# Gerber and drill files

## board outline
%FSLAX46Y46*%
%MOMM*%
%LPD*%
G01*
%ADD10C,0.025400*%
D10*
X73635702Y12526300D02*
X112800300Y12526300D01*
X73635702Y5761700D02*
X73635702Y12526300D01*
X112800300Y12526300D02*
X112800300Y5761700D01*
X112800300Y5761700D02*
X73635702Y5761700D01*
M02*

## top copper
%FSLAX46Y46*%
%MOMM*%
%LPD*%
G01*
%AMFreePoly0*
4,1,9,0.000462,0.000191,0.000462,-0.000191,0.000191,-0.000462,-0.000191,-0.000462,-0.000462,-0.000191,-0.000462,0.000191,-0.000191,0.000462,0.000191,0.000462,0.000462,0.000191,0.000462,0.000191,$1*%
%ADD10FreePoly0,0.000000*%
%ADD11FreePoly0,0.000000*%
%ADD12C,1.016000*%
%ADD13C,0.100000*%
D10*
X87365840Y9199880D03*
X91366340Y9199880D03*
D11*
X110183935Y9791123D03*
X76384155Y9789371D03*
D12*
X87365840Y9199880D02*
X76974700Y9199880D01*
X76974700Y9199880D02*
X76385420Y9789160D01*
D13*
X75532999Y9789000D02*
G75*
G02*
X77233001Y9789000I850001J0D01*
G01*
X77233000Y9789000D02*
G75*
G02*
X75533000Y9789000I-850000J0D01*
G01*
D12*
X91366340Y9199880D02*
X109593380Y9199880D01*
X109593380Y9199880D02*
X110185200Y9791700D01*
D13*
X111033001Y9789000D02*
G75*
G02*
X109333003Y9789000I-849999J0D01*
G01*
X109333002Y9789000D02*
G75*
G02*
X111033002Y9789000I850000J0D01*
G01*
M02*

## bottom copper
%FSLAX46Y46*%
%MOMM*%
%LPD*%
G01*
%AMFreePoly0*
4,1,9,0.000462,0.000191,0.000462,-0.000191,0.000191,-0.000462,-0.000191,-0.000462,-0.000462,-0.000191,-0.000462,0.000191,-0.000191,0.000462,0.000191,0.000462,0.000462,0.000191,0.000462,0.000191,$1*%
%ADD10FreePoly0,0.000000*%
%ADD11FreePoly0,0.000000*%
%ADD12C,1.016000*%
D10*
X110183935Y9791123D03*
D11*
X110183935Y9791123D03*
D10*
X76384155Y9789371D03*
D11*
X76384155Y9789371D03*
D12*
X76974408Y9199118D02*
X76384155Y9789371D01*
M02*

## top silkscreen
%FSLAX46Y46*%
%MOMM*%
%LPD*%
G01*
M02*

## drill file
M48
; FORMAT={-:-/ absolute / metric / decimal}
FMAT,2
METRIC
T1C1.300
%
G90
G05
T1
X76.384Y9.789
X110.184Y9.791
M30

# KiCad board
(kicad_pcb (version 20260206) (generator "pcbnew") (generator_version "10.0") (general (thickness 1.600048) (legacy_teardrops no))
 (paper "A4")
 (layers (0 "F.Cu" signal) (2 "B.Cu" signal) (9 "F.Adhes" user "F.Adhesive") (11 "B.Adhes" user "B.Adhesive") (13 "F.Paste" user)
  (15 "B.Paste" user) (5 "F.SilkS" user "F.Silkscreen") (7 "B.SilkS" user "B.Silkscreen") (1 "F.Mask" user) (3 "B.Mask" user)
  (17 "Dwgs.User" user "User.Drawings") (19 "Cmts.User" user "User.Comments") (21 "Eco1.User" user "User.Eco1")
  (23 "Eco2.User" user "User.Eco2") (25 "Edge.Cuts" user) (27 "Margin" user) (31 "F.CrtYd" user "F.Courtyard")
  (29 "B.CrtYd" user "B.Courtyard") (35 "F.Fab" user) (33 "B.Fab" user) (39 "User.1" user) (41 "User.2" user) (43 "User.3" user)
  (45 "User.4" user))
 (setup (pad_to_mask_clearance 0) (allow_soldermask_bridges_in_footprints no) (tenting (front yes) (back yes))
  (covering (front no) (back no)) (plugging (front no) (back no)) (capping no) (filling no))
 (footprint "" (layer "F.Cu") (at 0 0)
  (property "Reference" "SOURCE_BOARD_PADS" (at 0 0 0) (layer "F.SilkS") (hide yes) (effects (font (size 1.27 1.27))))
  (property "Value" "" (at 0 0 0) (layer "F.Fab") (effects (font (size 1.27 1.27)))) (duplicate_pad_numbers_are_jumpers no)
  (pad "1" smd custom (at 87.36584 -9.19988) (size 0.001 0.001) (layers "F.Cu" "F.Mask" "F.Paste") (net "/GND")
   (options (clearance outline) (anchor circle)) (primitives))
  (pad "2" smd custom (at 91.36634 -9.19988) (size 0.001 0.001) (layers "F.Cu" "F.Mask" "F.Paste") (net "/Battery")
   (options (clearance outline) (anchor circle)) (primitives)))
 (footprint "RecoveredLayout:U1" (layer "B.Cu") (at 110.183935 -9.791123)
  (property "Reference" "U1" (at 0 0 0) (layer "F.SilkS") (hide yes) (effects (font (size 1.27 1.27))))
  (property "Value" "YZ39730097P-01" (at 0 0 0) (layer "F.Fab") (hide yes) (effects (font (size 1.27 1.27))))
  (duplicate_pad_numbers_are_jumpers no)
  (pad "1" thru_hole custom (at 0 0) (size 0.001 0.001) (drill 1.300023) (layers "*.Cu") (remove_unused_layers no) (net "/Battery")
   (options (clearance outline) (anchor circle)) (primitives))
  (pad "1" smd custom (at 0 0) (size 0.001 0.001) (layers "B.Cu" "B.Mask" "B.Paste") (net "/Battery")
   (options (clearance outline) (anchor circle)) (primitives)))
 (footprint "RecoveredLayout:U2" (layer "B.Cu") (at 76.384155 -9.789371)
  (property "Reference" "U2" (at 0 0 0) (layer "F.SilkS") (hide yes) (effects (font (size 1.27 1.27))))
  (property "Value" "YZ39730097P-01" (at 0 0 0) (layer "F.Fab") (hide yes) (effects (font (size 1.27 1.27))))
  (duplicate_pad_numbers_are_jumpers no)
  (pad "1" thru_hole custom (at 0 0) (size 0.001 0.001) (drill 1.300023) (layers "*.Cu") (remove_unused_layers no) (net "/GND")
   (options (clearance outline) (anchor circle)) (primitives))
  (pad "1" smd custom (at 0 0) (size 0.001 0.001) (layers "B.Cu" "B.Mask" "B.Paste") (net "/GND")
   (options (clearance outline) (anchor circle)) (primitives)))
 (gr_line (start 73.635702 -12.5263) (end 112.8003 -12.5263) (stroke (width 0.0254) (type default)) (layer "Edge.Cuts"))
 (gr_line (start 73.635702 -5.7617) (end 73.635702 -12.5263) (stroke (width 0.0254) (type default)) (layer "Edge.Cuts"))
 (gr_line (start 112.8003 -12.5263) (end 112.8003 -5.7617) (stroke (width 0.0254) (type default)) (layer "Edge.Cuts"))
 (gr_line (start 112.8003 -5.7617) (end 73.635702 -5.7617) (stroke (width 0.0254) (type default)) (layer "Edge.Cuts"))
 (segment (start 87.36584 -9.19988) (end 76.9747 -9.19988) (width 1.016) (layer "F.Cu") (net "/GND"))
 (segment (start 76.9747 -9.19988) (end 76.38542 -9.78916) (width 1.016) (layer "F.Cu") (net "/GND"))
 (arc (start 75.532999 -9.789) (mid 76.401288 -10.638804) (end 77.233 -9.789) (width 0.1) (layer "F.Cu") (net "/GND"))
 (arc (start 77.233 -9.789) (mid 76.364711 -8.939196) (end 75.532999 -9.789) (width 0.1) (layer "F.Cu") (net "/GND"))
 (segment (start 76.974408 -9.199118) (end 76.384155 -9.789371) (width 1.016) (layer "B.Cu") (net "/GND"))
 (segment (start 91.36634 -9.19988) (end 109.59338 -9.19988) (width 1.016) (layer "F.Cu") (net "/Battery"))
 (segment (start 109.59338 -9.19988) (end 110.1852 -9.7917) (width 1.016) (layer "F.Cu") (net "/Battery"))
 (arc (start 111.033001 -9.789) (mid 110.164713 -8.939197) (end 109.333002 -9.789) (width 0.1) (layer "F.Cu") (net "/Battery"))
 (arc (start 109.333002 -9.789) (mid 110.20129 -10.638803) (end 111.033001 -9.789) (width 0.1) (layer "F.Cu") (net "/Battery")))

